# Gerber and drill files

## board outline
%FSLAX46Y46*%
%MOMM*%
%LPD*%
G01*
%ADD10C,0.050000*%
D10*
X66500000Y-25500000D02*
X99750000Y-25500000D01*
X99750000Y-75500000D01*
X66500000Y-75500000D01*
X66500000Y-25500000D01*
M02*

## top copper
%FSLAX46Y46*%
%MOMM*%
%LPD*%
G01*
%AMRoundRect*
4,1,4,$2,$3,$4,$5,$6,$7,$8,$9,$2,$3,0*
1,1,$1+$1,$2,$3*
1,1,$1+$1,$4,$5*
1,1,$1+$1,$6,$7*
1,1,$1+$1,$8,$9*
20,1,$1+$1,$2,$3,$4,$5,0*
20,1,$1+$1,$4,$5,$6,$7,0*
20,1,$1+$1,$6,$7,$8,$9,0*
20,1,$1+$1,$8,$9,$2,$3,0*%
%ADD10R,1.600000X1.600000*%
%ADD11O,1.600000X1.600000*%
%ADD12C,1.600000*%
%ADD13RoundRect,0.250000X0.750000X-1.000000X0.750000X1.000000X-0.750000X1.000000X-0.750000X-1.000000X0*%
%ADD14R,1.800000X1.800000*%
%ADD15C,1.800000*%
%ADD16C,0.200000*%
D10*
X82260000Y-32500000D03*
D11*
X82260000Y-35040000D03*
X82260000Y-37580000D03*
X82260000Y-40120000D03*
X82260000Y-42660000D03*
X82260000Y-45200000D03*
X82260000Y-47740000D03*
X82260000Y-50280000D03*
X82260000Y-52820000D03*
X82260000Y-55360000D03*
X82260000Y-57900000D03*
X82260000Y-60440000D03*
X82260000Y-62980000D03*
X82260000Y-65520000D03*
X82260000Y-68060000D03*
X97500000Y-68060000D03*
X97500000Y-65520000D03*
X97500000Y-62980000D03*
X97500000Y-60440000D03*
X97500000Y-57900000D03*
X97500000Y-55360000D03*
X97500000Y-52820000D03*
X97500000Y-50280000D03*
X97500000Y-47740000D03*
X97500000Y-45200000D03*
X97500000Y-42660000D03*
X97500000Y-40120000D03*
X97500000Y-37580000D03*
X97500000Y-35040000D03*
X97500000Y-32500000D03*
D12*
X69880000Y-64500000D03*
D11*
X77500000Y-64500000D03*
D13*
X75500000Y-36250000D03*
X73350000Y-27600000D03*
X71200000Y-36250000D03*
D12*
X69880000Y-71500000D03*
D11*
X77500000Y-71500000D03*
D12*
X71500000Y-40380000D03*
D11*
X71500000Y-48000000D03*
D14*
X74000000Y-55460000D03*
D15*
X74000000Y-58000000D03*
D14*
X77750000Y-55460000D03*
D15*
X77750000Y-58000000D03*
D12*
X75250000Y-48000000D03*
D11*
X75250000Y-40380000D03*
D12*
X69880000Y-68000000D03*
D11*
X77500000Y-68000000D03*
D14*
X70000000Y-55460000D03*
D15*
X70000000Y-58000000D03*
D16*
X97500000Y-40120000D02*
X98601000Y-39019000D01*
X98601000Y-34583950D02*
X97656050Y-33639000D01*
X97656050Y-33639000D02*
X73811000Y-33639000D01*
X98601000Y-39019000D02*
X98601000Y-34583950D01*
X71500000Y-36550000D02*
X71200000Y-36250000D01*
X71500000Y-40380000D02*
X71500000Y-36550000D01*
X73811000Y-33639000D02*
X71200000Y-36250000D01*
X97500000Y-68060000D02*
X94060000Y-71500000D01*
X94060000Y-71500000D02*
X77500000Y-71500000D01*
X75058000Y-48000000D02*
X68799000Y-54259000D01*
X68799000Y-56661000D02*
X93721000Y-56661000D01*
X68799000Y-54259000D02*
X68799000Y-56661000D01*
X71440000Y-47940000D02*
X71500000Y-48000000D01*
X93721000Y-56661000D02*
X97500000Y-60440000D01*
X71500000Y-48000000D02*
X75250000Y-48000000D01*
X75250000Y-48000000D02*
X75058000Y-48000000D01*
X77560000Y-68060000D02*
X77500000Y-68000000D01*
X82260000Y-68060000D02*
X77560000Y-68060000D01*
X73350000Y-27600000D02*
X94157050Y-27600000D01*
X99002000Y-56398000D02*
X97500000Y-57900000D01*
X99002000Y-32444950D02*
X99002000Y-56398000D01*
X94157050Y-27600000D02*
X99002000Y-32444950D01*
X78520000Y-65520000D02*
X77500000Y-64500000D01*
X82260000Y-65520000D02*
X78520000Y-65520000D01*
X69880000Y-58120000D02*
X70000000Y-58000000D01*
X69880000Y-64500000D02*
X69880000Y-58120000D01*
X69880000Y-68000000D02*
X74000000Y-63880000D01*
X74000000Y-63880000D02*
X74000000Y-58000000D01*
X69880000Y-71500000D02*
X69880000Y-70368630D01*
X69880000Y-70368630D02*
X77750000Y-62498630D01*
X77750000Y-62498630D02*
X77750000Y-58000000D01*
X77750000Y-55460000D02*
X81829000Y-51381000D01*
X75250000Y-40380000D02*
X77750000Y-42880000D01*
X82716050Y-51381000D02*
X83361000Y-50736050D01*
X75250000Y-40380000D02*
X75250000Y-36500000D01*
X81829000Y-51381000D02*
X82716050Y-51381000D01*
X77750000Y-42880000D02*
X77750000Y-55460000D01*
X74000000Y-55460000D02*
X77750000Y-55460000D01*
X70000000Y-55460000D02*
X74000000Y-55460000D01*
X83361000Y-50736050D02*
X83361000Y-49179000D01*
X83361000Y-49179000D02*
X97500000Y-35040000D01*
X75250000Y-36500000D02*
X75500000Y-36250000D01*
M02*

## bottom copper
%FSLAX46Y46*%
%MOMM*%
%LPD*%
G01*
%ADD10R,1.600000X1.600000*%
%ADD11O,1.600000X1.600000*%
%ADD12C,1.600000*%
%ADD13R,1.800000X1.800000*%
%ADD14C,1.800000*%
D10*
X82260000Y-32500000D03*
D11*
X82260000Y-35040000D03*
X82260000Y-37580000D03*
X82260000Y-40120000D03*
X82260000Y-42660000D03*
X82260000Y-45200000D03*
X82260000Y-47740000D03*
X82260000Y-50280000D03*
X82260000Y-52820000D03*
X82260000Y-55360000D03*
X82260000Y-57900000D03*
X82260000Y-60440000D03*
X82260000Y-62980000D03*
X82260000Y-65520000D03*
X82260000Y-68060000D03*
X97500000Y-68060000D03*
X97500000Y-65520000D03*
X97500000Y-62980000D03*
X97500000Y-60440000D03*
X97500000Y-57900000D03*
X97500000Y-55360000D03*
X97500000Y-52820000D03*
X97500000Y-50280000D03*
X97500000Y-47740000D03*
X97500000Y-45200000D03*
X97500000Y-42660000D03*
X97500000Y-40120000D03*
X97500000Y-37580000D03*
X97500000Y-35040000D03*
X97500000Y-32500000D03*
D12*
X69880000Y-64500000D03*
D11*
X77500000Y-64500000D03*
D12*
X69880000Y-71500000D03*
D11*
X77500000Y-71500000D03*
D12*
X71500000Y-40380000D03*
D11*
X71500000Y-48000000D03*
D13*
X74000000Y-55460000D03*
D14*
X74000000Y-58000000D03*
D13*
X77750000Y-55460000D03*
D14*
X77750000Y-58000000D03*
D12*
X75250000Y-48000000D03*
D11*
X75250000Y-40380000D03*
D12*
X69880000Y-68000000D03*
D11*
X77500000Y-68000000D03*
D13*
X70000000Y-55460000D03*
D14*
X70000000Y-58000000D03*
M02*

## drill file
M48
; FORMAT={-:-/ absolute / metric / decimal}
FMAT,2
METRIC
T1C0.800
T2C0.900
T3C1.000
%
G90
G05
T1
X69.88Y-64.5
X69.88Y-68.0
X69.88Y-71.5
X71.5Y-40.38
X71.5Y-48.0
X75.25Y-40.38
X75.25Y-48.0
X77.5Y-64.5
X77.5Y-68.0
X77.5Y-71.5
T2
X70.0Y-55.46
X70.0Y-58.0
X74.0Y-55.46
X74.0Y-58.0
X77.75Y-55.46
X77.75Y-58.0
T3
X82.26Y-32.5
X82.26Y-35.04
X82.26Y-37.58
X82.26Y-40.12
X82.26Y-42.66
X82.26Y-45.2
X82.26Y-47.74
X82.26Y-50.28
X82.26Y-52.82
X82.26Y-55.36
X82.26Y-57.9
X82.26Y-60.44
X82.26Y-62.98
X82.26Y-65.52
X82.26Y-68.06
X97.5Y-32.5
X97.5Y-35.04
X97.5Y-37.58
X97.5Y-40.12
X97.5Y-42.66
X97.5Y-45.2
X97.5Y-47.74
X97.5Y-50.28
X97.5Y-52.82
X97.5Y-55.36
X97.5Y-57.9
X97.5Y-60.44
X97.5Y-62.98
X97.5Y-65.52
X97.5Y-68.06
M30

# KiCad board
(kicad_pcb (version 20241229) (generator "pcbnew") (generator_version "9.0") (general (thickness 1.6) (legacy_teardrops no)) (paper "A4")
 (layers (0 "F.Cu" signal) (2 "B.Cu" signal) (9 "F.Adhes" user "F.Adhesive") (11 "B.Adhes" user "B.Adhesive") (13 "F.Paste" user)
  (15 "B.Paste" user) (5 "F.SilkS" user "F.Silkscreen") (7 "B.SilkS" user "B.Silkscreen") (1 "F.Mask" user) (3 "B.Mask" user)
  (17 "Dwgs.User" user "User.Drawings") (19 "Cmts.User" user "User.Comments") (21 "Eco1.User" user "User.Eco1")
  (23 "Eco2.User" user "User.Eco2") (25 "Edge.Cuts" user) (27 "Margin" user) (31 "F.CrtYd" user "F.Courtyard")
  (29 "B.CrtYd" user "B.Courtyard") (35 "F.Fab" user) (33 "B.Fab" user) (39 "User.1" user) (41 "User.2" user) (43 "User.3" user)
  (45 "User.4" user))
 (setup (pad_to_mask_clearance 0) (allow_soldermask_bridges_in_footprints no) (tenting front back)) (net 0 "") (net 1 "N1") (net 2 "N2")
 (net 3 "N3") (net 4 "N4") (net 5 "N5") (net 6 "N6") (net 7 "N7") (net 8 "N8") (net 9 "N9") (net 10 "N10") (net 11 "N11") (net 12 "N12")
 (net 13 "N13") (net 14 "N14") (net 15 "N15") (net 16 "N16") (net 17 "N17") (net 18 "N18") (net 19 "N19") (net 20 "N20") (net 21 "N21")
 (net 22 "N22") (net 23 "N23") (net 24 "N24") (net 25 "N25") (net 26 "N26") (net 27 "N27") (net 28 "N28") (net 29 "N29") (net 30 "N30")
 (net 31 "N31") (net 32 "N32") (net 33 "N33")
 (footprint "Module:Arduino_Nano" (layer "F.Cu") (at 82.26 32.5)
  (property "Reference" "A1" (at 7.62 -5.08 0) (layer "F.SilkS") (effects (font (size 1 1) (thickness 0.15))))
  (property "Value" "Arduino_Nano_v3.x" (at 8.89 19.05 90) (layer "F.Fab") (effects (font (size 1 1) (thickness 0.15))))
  (pad "1" thru_hole rect (at 0 0) (size 1.6 1.6) (drill 1) (layers "*.Cu" "*.Mask") (remove_unused_layers no) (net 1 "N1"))
  (pad "2" thru_hole oval (at 0 2.54) (size 1.6 1.6) (drill 1) (layers "*.Cu" "*.Mask") (remove_unused_layers no) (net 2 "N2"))
  (pad "3" thru_hole oval (at 0 5.08) (size 1.6 1.6) (drill 1) (layers "*.Cu" "*.Mask") (remove_unused_layers no) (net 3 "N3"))
  (pad "4" thru_hole oval (at 0 7.62) (size 1.6 1.6) (drill 1) (layers "*.Cu" "*.Mask") (remove_unused_layers no) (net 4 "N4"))
  (pad "5" thru_hole oval (at 0 10.16) (size 1.6 1.6) (drill 1) (layers "*.Cu" "*.Mask") (remove_unused_layers no) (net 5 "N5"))
  (pad "6" thru_hole oval (at 0 12.7) (size 1.6 1.6) (drill 1) (layers "*.Cu" "*.Mask") (remove_unused_layers no) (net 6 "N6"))
  (pad "7" thru_hole oval (at 0 15.24) (size 1.6 1.6) (drill 1) (layers "*.Cu" "*.Mask") (remove_unused_layers no) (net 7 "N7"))
  (pad "8" thru_hole oval (at 0 17.78) (size 1.6 1.6) (drill 1) (layers "*.Cu" "*.Mask") (remove_unused_layers no) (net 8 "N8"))
  (pad "9" thru_hole oval (at 0 20.32) (size 1.6 1.6) (drill 1) (layers "*.Cu" "*.Mask") (remove_unused_layers no) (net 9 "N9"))
  (pad "10" thru_hole oval (at 0 22.86) (size 1.6 1.6) (drill 1) (layers "*.Cu" "*.Mask") (remove_unused_layers no) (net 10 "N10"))
  (pad "11" thru_hole oval (at 0 25.4) (size 1.6 1.6) (drill 1) (layers "*.Cu" "*.Mask") (remove_unused_layers no) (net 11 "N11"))
  (pad "12" thru_hole oval (at 0 27.94) (size 1.6 1.6) (drill 1) (layers "*.Cu" "*.Mask") (remove_unused_layers no) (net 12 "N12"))
  (pad "13" thru_hole oval (at 0 30.48) (size 1.6 1.6) (drill 1) (layers "*.Cu" "*.Mask") (remove_unused_layers no) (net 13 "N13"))
  (pad "14" thru_hole oval (at 0 33.02) (size 1.6 1.6) (drill 1) (layers "*.Cu" "*.Mask") (remove_unused_layers no) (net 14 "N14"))
  (pad "15" thru_hole oval (at 0 35.56) (size 1.6 1.6) (drill 1) (layers "*.Cu" "*.Mask") (remove_unused_layers no) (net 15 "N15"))
  (pad "16" thru_hole oval (at 15.24 35.56) (size 1.6 1.6) (drill 1) (layers "*.Cu" "*.Mask") (remove_unused_layers no) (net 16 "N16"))
  (pad "17" thru_hole oval (at 15.24 33.02) (size 1.6 1.6) (drill 1) (layers "*.Cu" "*.Mask") (remove_unused_layers no) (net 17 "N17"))
  (pad "18" thru_hole oval (at 15.24 30.48) (size 1.6 1.6) (drill 1) (layers "*.Cu" "*.Mask") (remove_unused_layers no) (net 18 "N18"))
  (pad "19" thru_hole oval (at 15.24 27.94) (size 1.6 1.6) (drill 1) (layers "*.Cu" "*.Mask") (remove_unused_layers no) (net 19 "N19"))
  (pad "20" thru_hole oval (at 15.24 25.4) (size 1.6 1.6) (drill 1) (layers "*.Cu" "*.Mask") (remove_unused_layers no) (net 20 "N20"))
  (pad "21" thru_hole oval (at 15.24 22.86) (size 1.6 1.6) (drill 1) (layers "*.Cu" "*.Mask") (remove_unused_layers no) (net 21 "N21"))
  (pad "22" thru_hole oval (at 15.24 20.32) (size 1.6 1.6) (drill 1) (layers "*.Cu" "*.Mask") (remove_unused_layers no) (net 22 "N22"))
  (pad "23" thru_hole oval (at 15.24 17.78) (size 1.6 1.6) (drill 1) (layers "*.Cu" "*.Mask") (remove_unused_layers no) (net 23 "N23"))
  (pad "24" thru_hole oval (at 15.24 15.24) (size 1.6 1.6) (drill 1) (layers "*.Cu" "*.Mask") (remove_unused_layers no) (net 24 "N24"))
  (pad "25" thru_hole oval (at 15.24 12.7) (size 1.6 1.6) (drill 1) (layers "*.Cu" "*.Mask") (remove_unused_layers no) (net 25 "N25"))
  (pad "26" thru_hole oval (at 15.24 10.16) (size 1.6 1.6) (drill 1) (layers "*.Cu" "*.Mask") (remove_unused_layers no) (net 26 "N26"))
  (pad "27" thru_hole oval (at 15.24 7.62) (size 1.6 1.6) (drill 1) (layers "*.Cu" "*.Mask") (remove_unused_layers no) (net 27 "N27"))
  (pad "28" thru_hole oval (at 15.24 5.08) (size 1.6 1.6) (drill 1) (layers "*.Cu" "*.Mask") (remove_unused_layers no) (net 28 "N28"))
  (pad "29" thru_hole oval (at 15.24 2.54) (size 1.6 1.6) (drill 1) (layers "*.Cu" "*.Mask") (remove_unused_layers no) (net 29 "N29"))
  (pad "30" thru_hole oval (at 15.24 0) (size 1.6 1.6) (drill 1) (layers "*.Cu" "*.Mask") (remove_unused_layers no) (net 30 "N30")))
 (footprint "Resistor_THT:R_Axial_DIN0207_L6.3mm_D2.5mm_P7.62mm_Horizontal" (layer "F.Cu") (at 69.88 64.5)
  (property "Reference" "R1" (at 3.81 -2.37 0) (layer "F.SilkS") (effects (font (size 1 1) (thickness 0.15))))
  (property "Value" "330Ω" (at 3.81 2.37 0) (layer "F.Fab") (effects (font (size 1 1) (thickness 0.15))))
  (pad "1" thru_hole circle (at 0 0) (size 1.6 1.6) (drill 0.8) (layers "*.Cu" "*.Mask") (remove_unused_layers no) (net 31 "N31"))
  (pad "2" thru_hole oval (at 7.62 0) (size 1.6 1.6) (drill 0.8) (layers "*.Cu" "*.Mask") (remove_unused_layers no) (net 14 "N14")))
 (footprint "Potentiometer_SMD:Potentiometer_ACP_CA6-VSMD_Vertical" (layer "F.Cu") (at 73.35 31.925 90)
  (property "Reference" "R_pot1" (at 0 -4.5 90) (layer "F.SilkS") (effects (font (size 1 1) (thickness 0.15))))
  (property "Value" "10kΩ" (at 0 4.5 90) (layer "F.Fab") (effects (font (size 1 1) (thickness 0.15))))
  (pad "1" smd roundrect (at -4.325 2.15 90) (size 2.5 2) (layers "F.Cu" "F.Mask" "F.Paste") (roundrect_rratio 0.125) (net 29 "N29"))
  (pad "2" smd roundrect (at 4.325 0 90) (size 2.5 2) (layers "F.Cu" "F.Mask" "F.Paste") (roundrect_rratio 0.125) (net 20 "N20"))
  (pad "3" smd roundrect (at -4.325 -2.15 90) (size 2.5 2) (layers "F.Cu" "F.Mask" "F.Paste") (roundrect_rratio 0.125) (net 27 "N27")))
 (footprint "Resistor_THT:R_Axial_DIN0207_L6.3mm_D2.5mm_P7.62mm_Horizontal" (layer "F.Cu") (at 69.88 71.5)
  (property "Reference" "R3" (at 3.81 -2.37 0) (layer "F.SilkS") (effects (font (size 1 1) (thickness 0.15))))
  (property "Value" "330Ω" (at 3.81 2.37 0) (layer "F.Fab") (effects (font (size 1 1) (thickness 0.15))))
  (pad "1" thru_hole circle (at 0 0) (size 1.6 1.6) (drill 0.8) (layers "*.Cu" "*.Mask") (remove_unused_layers no) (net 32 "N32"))
  (pad "2" thru_hole oval (at 7.62 0) (size 1.6 1.6) (drill 0.8) (layers "*.Cu" "*.Mask") (remove_unused_layers no) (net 16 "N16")))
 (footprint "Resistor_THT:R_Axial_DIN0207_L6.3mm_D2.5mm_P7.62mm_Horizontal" (layer "F.Cu") (at 71.5 40.38 -90)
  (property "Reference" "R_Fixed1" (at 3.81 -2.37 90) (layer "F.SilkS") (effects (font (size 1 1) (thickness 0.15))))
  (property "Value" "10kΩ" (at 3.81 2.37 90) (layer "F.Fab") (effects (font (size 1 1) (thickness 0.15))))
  (pad "1" thru_hole circle (at 0 0 270) (size 1.6 1.6) (drill 0.8) (layers "*.Cu" "*.Mask") (remove_unused_layers no) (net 27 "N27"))
  (pad "2" thru_hole oval (at 7.62 0 270) (size 1.6 1.6) (drill 0.8) (layers "*.Cu" "*.Mask") (remove_unused_layers no) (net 19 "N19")))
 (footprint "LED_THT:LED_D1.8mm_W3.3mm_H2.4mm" (layer "F.Cu") (at 74 55.46 -90)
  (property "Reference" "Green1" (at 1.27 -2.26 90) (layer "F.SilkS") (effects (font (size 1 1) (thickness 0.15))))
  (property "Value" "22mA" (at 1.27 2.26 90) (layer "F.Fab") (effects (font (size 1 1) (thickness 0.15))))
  (pad "1" thru_hole rect (at 0 0 270) (size 1.8 1.8) (drill 0.9) (layers "*.Cu" "*.Mask") (remove_unused_layers no) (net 29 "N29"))
  (pad "2" thru_hole circle (at 2.54 0 270) (size 1.8 1.8) (drill 0.9) (layers "*.Cu" "*.Mask") (remove_unused_layers no) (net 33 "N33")))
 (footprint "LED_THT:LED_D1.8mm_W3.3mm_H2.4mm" (layer "F.Cu") (at 77.75 55.46 -90)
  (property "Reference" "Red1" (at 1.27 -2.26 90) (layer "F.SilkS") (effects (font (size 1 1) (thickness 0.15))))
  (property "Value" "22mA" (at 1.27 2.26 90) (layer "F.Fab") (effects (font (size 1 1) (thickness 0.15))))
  (pad "1" thru_hole rect (at 0 0 270) (size 1.8 1.8) (drill 0.9) (layers "*.Cu" "*.Mask") (remove_unused_layers no) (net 29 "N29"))
  (pad "2" thru_hole circle (at 2.54 0 270) (size 1.8 1.8) (drill 0.9) (layers "*.Cu" "*.Mask") (remove_unused_layers no) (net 32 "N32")))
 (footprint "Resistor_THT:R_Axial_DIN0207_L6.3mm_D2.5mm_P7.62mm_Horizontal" (layer "F.Cu") (at 75.25 48 90)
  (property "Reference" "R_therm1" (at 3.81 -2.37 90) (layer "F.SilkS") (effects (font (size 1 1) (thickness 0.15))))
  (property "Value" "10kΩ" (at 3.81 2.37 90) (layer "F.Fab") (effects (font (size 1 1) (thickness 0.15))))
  (pad "1" thru_hole circle (at 0 0 90) (size 1.6 1.6) (drill 0.8) (layers "*.Cu" "*.Mask") (remove_unused_layers no) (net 19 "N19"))
  (pad "2" thru_hole oval (at 7.62 0 90) (size 1.6 1.6) (drill 0.8) (layers "*.Cu" "*.Mask") (remove_unused_layers no) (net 29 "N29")))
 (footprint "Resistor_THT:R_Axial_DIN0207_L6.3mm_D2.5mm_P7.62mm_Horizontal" (layer "F.Cu") (at 69.88 68)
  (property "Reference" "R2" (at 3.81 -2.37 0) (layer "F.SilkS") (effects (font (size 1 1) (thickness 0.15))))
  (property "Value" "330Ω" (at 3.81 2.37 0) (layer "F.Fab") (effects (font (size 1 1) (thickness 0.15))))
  (pad "1" thru_hole circle (at 0 0) (size 1.6 1.6) (drill 0.8) (layers "*.Cu" "*.Mask") (remove_unused_layers no) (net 33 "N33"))
  (pad "2" thru_hole oval (at 7.62 0) (size 1.6 1.6) (drill 0.8) (layers "*.Cu" "*.Mask") (remove_unused_layers no) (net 15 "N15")))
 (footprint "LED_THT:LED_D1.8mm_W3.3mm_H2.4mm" (layer "F.Cu") (at 70 55.46 -90)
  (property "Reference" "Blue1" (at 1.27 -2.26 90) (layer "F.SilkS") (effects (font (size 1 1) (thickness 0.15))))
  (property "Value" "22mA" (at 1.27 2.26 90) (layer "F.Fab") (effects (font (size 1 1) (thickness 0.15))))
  (pad "1" thru_hole rect (at 0 0 270) (size 1.8 1.8) (drill 0.9) (layers "*.Cu" "*.Mask") (remove_unused_layers no) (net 29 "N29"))
  (pad "2" thru_hole circle (at 2.54 0 270) (size 1.8 1.8) (drill 0.9) (layers "*.Cu" "*.Mask") (remove_unused_layers no) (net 31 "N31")))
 (gr_rect (start 66.5 25.5) (end 99.75 75.5) (stroke (width 0.05) (type default)) (fill no) (layer "Edge.Cuts"))
 (segment (start 97.5 40.12) (end 98.601 39.019) (width 0.2) (layer "F.Cu") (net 27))
 (segment (start 98.601 34.58395) (end 97.65605 33.639) (width 0.2) (layer "F.Cu") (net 27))
 (segment (start 97.65605 33.639) (end 73.811 33.639) (width 0.2) (layer "F.Cu") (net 27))
 (segment (start 98.601 39.019) (end 98.601 34.58395) (width 0.2) (layer "F.Cu") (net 27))
 (segment (start 71.5 36.55) (end 71.2 36.25) (width 0.2) (layer "F.Cu") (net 27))
 (segment (start 71.5 40.38) (end 71.5 36.55) (width 0.2) (layer "F.Cu") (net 27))
 (segment (start 73.811 33.639) (end 71.2 36.25) (width 0.2) (layer "F.Cu") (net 27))
 (segment (start 97.5 68.06) (end 94.06 71.5) (width 0.2) (layer "F.Cu") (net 16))
 (segment (start 94.06 71.5) (end 77.5 71.5) (width 0.2) (layer "F.Cu") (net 16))
 (segment (start 75.058 48) (end 68.799 54.259) (width 0.2) (layer "F.Cu") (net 19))
 (segment (start 68.799 56.661) (end 93.721 56.661) (width 0.2) (layer "F.Cu") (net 19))
 (segment (start 68.799 54.259) (end 68.799 56.661) (width 0.2) (layer "F.Cu") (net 19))
 (segment (start 71.44 47.94) (end 71.5 48) (width 0.2) (layer "F.Cu") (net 19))
 (segment (start 93.721 56.661) (end 97.5 60.44) (width 0.2) (layer "F.Cu") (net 19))
 (segment (start 71.5 48) (end 75.25 48) (width 0.2) (layer "F.Cu") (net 19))
 (segment (start 75.25 48) (end 75.058 48) (width 0.2) (layer "F.Cu") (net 19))
 (segment (start 77.56 68.06) (end 77.5 68) (width 0.2) (layer "F.Cu") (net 15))
 (segment (start 82.26 68.06) (end 77.56 68.06) (width 0.2) (layer "F.Cu") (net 15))
 (segment (start 73.35 27.6) (end 94.15705 27.6) (width 0.2) (layer "F.Cu") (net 20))
 (segment (start 99.002 56.398) (end 97.5 57.9) (width 0.2) (layer "F.Cu") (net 20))
 (segment (start 99.002 32.44495) (end 99.002 56.398) (width 0.2) (layer "F.Cu") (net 20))
 (segment (start 94.15705 27.6) (end 99.002 32.44495) (width 0.2) (layer "F.Cu") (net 20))
 (segment (start 78.52 65.52) (end 77.5 64.5) (width 0.2) (layer "F.Cu") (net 14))
 (segment (start 82.26 65.52) (end 78.52 65.52) (width 0.2) (layer "F.Cu") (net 14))
 (segment (start 69.88 58.12) (end 70 58) (width 0.2) (layer "F.Cu") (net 31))
 (segment (start 69.88 64.5) (end 69.88 58.12) (width 0.2) (layer "F.Cu") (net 31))
 (segment (start 69.88 68) (end 74 63.88) (width 0.2) (layer "F.Cu") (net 33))
 (segment (start 74 63.88) (end 74 58) (width 0.2) (layer "F.Cu") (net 33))
 (segment (start 69.88 71.5) (end 69.88 70.36863) (width 0.2) (layer "F.Cu") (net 32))
 (segment (start 69.88 70.36863) (end 77.75 62.49863) (width 0.2) (layer "F.Cu") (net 32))
 (segment (start 77.75 62.49863) (end 77.75 58) (width 0.2) (layer "F.Cu") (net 32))
 (segment (start 77.75 55.46) (end 81.829 51.381) (width 0.2) (layer "F.Cu") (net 29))
 (segment (start 75.25 40.38) (end 77.75 42.88) (width 0.2) (layer "F.Cu") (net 29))
 (segment (start 82.71605 51.381) (end 83.361 50.73605) (width 0.2) (layer "F.Cu") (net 29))
 (segment (start 75.25 40.38) (end 75.25 36.5) (width 0.2) (layer "F.Cu") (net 29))
 (segment (start 81.829 51.381) (end 82.71605 51.381) (width 0.2) (layer "F.Cu") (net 29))
 (segment (start 77.75 42.88) (end 77.75 55.46) (width 0.2) (layer "F.Cu") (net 29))
 (segment (start 74 55.46) (end 77.75 55.46) (width 0.2) (layer "F.Cu") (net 29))
 (segment (start 70 55.46) (end 74 55.46) (width 0.2) (layer "F.Cu") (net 29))
 (segment (start 83.361 50.73605) (end 83.361 49.179) (width 0.2) (layer "F.Cu") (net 29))
 (segment (start 83.361 49.179) (end 97.5 35.04) (width 0.2) (layer "F.Cu") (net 29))
 (segment (start 75.25 36.5) (end 75.5 36.25) (width 0.2) (layer "F.Cu") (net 29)))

